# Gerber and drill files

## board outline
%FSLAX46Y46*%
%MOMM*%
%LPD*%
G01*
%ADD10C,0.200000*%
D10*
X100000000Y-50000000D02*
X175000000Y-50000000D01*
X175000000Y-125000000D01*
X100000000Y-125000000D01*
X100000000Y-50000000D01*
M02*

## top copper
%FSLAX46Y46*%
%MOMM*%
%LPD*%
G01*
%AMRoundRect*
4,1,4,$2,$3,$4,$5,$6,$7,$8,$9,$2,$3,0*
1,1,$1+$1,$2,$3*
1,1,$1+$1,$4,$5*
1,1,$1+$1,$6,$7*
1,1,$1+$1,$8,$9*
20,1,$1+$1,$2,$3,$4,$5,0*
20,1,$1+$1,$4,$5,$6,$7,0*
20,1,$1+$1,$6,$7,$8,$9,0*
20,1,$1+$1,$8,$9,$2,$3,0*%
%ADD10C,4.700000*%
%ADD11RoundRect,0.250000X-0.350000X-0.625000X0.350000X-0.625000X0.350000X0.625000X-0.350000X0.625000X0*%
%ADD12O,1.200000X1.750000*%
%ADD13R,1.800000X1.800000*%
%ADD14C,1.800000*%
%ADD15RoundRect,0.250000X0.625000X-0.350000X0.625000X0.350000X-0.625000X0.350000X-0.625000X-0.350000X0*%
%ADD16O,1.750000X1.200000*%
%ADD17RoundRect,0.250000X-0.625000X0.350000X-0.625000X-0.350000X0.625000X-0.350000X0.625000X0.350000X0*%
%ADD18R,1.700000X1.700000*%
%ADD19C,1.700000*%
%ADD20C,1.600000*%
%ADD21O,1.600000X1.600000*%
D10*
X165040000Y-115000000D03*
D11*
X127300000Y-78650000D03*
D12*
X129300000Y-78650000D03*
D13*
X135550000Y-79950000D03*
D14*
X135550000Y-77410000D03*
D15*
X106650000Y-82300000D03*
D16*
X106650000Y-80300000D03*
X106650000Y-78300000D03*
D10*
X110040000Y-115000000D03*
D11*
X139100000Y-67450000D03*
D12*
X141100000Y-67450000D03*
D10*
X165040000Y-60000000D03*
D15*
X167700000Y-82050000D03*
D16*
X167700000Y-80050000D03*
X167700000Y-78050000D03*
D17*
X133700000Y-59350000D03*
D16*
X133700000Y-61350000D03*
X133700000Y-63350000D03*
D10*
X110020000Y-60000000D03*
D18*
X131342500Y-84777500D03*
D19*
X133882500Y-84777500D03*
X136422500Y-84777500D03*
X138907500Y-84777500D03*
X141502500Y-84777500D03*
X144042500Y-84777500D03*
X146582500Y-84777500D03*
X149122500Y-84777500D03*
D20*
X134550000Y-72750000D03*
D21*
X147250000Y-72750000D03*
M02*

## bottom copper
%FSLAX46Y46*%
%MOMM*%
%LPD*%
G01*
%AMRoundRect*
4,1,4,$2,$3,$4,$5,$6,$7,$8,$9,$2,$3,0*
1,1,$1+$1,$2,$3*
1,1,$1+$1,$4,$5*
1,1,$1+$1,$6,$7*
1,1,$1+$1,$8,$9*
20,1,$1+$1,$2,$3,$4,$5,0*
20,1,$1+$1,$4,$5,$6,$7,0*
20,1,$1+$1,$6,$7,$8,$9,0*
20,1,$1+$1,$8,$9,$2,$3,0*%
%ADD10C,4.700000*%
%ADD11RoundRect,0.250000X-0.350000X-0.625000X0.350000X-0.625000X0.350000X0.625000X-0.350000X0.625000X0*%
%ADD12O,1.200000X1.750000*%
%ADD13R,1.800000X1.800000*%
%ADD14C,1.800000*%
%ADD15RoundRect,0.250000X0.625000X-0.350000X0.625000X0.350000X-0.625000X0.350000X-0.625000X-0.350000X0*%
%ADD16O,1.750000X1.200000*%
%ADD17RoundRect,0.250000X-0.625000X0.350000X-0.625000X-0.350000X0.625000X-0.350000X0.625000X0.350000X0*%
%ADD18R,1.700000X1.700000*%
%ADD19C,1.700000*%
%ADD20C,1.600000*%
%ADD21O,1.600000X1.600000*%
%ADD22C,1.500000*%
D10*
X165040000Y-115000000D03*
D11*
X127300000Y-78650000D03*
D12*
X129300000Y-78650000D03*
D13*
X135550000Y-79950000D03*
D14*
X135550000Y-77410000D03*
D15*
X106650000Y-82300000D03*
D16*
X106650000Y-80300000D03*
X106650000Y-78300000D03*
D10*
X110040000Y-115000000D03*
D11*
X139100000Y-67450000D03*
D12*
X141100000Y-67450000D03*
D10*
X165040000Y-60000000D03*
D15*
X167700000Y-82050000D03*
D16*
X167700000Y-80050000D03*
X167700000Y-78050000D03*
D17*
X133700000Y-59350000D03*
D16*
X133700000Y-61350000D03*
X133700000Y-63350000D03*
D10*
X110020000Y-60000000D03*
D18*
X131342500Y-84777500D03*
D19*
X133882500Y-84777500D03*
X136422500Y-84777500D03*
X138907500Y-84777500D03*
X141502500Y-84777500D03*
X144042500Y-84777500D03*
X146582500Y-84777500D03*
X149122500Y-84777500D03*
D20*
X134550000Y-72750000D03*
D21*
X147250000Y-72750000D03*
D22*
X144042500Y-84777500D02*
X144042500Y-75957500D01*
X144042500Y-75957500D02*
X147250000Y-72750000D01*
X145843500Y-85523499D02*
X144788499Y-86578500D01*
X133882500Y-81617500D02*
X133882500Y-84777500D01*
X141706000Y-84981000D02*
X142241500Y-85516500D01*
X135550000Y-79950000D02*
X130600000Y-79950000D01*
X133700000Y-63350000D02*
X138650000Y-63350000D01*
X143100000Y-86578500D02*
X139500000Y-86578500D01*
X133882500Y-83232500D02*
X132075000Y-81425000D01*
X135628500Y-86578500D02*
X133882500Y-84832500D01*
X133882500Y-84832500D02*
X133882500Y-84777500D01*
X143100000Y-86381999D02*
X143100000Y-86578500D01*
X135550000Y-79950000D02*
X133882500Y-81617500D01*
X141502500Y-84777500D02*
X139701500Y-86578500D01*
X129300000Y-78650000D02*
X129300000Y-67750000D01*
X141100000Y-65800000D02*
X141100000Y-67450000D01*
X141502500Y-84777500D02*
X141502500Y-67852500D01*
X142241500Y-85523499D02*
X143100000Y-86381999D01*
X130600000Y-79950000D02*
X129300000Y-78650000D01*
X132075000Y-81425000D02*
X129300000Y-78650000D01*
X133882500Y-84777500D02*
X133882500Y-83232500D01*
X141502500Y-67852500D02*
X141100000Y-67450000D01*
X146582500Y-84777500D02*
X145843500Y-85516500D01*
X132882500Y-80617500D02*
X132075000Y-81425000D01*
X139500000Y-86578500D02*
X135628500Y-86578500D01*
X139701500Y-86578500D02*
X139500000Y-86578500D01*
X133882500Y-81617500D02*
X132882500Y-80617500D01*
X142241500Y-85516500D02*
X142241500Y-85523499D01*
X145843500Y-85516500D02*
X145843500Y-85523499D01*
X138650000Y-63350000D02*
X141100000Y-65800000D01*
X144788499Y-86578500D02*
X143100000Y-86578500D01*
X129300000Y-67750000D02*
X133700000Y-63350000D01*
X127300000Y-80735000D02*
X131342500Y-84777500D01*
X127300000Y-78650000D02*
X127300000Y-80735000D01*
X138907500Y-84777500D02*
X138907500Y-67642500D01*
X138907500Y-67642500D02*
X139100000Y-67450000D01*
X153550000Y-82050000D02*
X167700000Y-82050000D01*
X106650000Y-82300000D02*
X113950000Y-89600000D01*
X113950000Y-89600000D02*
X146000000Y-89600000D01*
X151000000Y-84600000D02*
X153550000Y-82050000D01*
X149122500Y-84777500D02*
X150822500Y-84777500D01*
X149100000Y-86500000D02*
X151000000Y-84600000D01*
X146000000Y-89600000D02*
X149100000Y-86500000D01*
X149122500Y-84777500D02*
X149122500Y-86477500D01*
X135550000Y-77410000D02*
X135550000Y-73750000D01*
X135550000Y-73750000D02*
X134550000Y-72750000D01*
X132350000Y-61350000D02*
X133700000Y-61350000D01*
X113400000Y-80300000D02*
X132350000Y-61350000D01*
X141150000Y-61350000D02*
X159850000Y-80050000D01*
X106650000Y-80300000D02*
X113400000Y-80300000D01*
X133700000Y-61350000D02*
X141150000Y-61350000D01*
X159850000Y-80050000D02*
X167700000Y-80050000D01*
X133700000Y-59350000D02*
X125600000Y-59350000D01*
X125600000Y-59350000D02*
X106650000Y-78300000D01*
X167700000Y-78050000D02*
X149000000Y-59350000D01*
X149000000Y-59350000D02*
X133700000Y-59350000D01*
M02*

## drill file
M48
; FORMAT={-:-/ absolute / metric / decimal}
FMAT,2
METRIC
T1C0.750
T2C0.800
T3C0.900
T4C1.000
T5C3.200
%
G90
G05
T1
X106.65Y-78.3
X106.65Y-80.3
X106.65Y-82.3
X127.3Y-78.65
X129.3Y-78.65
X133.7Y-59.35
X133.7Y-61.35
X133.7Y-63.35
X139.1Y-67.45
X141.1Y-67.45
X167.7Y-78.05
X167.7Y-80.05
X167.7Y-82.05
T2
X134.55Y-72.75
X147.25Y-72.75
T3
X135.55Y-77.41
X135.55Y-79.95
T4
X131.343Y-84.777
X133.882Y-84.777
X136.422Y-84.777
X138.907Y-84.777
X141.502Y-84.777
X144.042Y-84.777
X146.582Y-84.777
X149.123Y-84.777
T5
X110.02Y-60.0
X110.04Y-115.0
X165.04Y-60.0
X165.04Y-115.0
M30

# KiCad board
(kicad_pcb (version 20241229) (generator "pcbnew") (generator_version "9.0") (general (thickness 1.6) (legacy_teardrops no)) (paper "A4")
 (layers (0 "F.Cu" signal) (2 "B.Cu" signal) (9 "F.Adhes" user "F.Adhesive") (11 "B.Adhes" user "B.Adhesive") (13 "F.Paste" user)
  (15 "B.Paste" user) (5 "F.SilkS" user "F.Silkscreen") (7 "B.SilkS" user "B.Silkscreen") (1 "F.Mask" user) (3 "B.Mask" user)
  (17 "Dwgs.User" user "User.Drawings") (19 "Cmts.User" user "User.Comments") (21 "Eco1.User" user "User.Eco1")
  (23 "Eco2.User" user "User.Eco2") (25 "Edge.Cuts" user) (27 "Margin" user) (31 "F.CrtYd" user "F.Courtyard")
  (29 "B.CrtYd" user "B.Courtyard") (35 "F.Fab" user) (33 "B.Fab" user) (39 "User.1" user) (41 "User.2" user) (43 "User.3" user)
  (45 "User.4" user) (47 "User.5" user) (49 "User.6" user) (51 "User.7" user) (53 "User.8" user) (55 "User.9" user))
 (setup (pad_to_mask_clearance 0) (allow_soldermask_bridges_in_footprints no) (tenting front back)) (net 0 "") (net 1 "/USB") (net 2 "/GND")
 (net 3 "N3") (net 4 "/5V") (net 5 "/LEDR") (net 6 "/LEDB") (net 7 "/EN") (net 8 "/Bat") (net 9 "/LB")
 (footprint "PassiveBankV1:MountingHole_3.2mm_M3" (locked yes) (layer "F.Cu") (at 165.02 115)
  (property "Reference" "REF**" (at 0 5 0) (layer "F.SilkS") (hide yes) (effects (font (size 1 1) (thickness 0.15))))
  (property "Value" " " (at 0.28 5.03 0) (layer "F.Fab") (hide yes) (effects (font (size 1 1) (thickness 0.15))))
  (pad "" np_thru_hole circle (at 0.02 0) (size 4.7 4.7) (drill 3.2) (layers "*.Cu" "*.Mask") (clearance 2)))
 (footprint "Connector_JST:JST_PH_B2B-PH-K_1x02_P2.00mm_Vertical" (layer "F.Cu") (at 127.3 78.65)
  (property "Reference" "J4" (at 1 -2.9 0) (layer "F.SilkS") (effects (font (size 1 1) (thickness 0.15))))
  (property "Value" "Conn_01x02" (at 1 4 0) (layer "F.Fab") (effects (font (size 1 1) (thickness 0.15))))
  (pad "1" thru_hole roundrect (at 0 0) (size 1.2 1.75) (drill 0.75) (layers "*.Cu" "*.Mask") (remove_unused_layers no)
   (roundrect_rratio 0.208333) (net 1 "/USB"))
  (pad "2" thru_hole oval (at 2 0) (size 1.2 1.75) (drill 0.75) (layers "*.Cu" "*.Mask") (remove_unused_layers no) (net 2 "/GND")))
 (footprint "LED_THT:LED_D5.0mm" (layer "F.Cu") (at 135.55 79.95 90)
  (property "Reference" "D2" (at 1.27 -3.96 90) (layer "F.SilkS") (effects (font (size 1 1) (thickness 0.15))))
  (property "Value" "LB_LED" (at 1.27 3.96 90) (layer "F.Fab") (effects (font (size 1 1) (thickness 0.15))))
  (pad "1" thru_hole rect (at 0 0 90) (size 1.8 1.8) (drill 0.9) (layers "*.Cu" "*.Mask") (remove_unused_layers no) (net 2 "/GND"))
  (pad "2" thru_hole circle (at 2.54 0 90) (size 1.8 1.8) (drill 0.9) (layers "*.Cu" "*.Mask") (remove_unused_layers no) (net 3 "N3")))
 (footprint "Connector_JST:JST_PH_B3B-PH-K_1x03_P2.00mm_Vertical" (layer "F.Cu") (at 106.65 82.3 90)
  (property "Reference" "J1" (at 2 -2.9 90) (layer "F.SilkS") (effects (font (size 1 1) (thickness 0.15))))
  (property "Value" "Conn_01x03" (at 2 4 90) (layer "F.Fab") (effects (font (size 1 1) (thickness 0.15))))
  (pad "1" thru_hole roundrect (at 0 0 90) (size 1.2 1.75) (drill 0.75) (layers "*.Cu" "*.Mask") (remove_unused_layers no)
   (roundrect_rratio 0.208333) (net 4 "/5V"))
  (pad "2" thru_hole oval (at 2 0 90) (size 1.2 1.75) (drill 0.75) (layers "*.Cu" "*.Mask") (remove_unused_layers no) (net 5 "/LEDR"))
  (pad "3" thru_hole oval (at 4 0 90) (size 1.2 1.75) (drill 0.75) (layers "*.Cu" "*.Mask") (remove_unused_layers no) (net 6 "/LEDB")))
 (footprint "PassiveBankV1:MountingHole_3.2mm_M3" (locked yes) (layer "F.Cu") (at 110.02 115)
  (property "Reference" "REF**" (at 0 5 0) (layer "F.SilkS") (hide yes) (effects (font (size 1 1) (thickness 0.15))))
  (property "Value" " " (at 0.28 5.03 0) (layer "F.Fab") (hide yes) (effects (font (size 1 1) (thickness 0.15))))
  (pad "" np_thru_hole circle (at 0.02 0) (size 4.7 4.7) (drill 3.2) (layers "*.Cu" "*.Mask") (clearance 2)))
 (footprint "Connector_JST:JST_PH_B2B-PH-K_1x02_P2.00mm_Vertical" (layer "F.Cu") (at 139.1 67.45)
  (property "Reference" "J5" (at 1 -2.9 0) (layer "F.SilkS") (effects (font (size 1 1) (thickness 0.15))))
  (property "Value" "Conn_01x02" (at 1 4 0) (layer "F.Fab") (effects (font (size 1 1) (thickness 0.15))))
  (pad "1" thru_hole roundrect (at 0 0) (size 1.2 1.75) (drill 0.75) (layers "*.Cu" "*.Mask") (remove_unused_layers no)
   (roundrect_rratio 0.208333) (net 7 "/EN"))
  (pad "2" thru_hole oval (at 2 0) (size 1.2 1.75) (drill 0.75) (layers "*.Cu" "*.Mask") (remove_unused_layers no) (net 2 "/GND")))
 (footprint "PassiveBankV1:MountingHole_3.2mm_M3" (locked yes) (layer "F.Cu") (at 165.02 60)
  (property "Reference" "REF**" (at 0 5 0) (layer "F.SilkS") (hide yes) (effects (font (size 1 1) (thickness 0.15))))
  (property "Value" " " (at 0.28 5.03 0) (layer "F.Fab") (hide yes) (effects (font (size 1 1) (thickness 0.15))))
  (pad "" np_thru_hole circle (at 0.02 0) (size 4.7 4.7) (drill 3.2) (layers "*.Cu" "*.Mask") (clearance 2)))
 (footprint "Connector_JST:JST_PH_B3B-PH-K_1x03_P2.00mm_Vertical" (layer "F.Cu") (at 167.7 82.05 90)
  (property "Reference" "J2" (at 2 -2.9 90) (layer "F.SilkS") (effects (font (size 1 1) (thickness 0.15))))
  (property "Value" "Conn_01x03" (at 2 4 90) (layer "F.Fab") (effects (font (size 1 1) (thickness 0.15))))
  (pad "1" thru_hole roundrect (at 0 0 90) (size 1.2 1.75) (drill 0.75) (layers "*.Cu" "*.Mask") (remove_unused_layers no)
   (roundrect_rratio 0.208333) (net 4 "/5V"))
  (pad "2" thru_hole oval (at 2 0 90) (size 1.2 1.75) (drill 0.75) (layers "*.Cu" "*.Mask") (remove_unused_layers no) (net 5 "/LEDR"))
  (pad "3" thru_hole oval (at 4 0 90) (size 1.2 1.75) (drill 0.75) (layers "*.Cu" "*.Mask") (remove_unused_layers no) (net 6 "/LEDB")))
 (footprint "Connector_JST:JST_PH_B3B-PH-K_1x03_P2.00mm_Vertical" (layer "F.Cu") (at 133.7 59.35 -90)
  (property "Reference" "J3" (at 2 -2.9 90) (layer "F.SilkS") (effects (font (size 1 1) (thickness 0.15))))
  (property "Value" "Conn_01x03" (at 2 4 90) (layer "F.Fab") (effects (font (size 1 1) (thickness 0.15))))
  (pad "1" thru_hole roundrect (at 0 0 270) (size 1.2 1.75) (drill 0.75) (layers "*.Cu" "*.Mask") (remove_unused_layers no)
   (roundrect_rratio 0.208333) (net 6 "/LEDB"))
  (pad "2" thru_hole oval (at 2 0 270) (size 1.2 1.75) (drill 0.75) (layers "*.Cu" "*.Mask") (remove_unused_layers no) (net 5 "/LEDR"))
  (pad "3" thru_hole oval (at 4 0 270) (size 1.2 1.75) (drill 0.75) (layers "*.Cu" "*.Mask") (remove_unused_layers no) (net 2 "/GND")))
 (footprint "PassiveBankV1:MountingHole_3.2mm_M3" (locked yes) (layer "F.Cu") (at 110 60)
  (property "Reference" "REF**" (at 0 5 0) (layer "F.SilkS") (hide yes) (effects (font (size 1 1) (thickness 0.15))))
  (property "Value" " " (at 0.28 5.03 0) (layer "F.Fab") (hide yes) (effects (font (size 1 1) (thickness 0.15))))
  (pad "" np_thru_hole circle (at 0.02 0) (size 4.7 4.7) (drill 3.2) (layers "*.Cu" "*.Mask") (clearance 2)))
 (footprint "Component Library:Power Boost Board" (layer "F.Cu") (at 149.1225 84.7775 -90)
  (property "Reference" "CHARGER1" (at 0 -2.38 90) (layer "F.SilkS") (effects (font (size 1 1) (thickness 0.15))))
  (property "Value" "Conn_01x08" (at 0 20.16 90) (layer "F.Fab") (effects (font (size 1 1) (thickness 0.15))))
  (pad "1" thru_hole rect (at 0 17.78 270) (size 1.7 1.7) (drill 1) (layers "*.Cu" "*.Mask") (remove_unused_layers no) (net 1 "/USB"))
  (pad "2" thru_hole circle (at 0 15.24 270) (size 1.7 1.7) (drill 1) (layers "*.Cu" "*.Mask") (remove_unused_layers no) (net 2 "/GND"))
  (pad "3" thru_hole circle (at 0 12.7 270) (size 1.7 1.7) (drill 1) (layers "*.Cu" "*.Mask") (remove_unused_layers no) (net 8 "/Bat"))
  (pad "4" thru_hole circle (at 0 10.215 270) (size 1.7 1.7) (drill 1) (layers "*.Cu" "*.Mask") (remove_unused_layers no) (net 7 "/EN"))
  (pad "5" thru_hole circle (at 0 7.62 270) (size 1.7 1.7) (drill 1) (layers "*.Cu" "*.Mask") (remove_unused_layers no) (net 2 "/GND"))
  (pad "6" thru_hole circle (at 0 5.08 270) (size 1.7 1.7) (drill 1) (layers "*.Cu" "*.Mask") (remove_unused_layers no) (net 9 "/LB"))
  (pad "7" thru_hole circle (at 0 2.54 270) (size 1.7 1.7) (drill 1) (layers "*.Cu" "*.Mask") (remove_unused_layers no) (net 2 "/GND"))
  (pad "8" thru_hole circle (at 0 0 270) (size 1.7 1.7) (drill 1) (layers "*.Cu" "*.Mask") (remove_unused_layers no) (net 4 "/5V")))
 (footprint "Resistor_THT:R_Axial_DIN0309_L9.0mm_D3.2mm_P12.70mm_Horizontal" (layer "F.Cu") (at 134.55 72.75)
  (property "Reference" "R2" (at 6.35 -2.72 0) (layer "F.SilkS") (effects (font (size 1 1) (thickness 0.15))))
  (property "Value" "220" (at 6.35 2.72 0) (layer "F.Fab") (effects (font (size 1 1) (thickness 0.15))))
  (pad "1" thru_hole circle (at 0 0) (size 1.6 1.6) (drill 0.8) (layers "*.Cu" "*.Mask") (remove_unused_layers no) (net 3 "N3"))
  (pad "2" thru_hole oval (at 12.7 0) (size 1.6 1.6) (drill 0.8) (layers "*.Cu" "*.Mask") (remove_unused_layers no) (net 9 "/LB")))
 (gr_rect (start 100 50) (end 175 125) (stroke (width 0.2) (type default)) (fill no) (locked yes) (layer "Edge.Cuts"))
 (segment (start 144.0425 84.7775) (end 144.0425 75.9575) (width 1.5) (layer "B.Cu") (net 9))
 (segment (start 144.0425 75.9575) (end 147.25 72.75) (width 1.5) (layer "B.Cu") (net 9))
 (segment (start 145.8435 85.523499) (end 144.788499 86.5785) (width 1.5) (layer "B.Cu") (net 2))
 (segment (start 133.8825 81.6175) (end 133.8825 84.7775) (width 1.5) (layer "B.Cu") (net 2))
 (segment (start 141.706 84.981) (end 142.2415 85.5165) (width 1.5) (layer "B.Cu") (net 2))
 (segment (start 135.55 79.95) (end 130.6 79.95) (width 1.5) (layer "B.Cu") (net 2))
 (segment (start 133.7 63.35) (end 138.65 63.35) (width 1.5) (layer "B.Cu") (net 2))
 (segment (start 143.1 86.5785) (end 139.5 86.5785) (width 1.5) (layer "B.Cu") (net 2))
 (segment (start 133.8825 83.2325) (end 132.075 81.425) (width 1.5) (layer "B.Cu") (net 2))
 (segment (start 135.6285 86.5785) (end 133.8825 84.8325) (width 1.5) (layer "B.Cu") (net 2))
 (segment (start 133.8825 84.8325) (end 133.8825 84.7775) (width 1.5) (layer "B.Cu") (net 2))
 (segment (start 143.1 86.381999) (end 143.1 86.5785) (width 1.5) (layer "B.Cu") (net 2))
 (segment (start 135.55 79.95) (end 133.8825 81.6175) (width 1.5) (layer "B.Cu") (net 2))
 (segment (start 141.5025 84.7775) (end 139.7015 86.5785) (width 1.5) (layer "B.Cu") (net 2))
 (segment (start 129.3 78.65) (end 129.3 67.75) (width 1.5) (layer "B.Cu") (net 2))
 (segment (start 141.1 65.8) (end 141.1 67.45) (width 1.5) (layer "B.Cu") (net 2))
 (segment (start 141.5025 84.7775) (end 141.5025 67.8525) (width 1.5) (layer "B.Cu") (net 2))
 (segment (start 142.2415 85.523499) (end 143.1 86.381999) (width 1.5) (layer "B.Cu") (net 2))
 (segment (start 130.6 79.95) (end 129.3 78.65) (width 1.5) (layer "B.Cu") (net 2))
 (segment (start 132.075 81.425) (end 129.3 78.65) (width 1.5) (layer "B.Cu") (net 2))
 (segment (start 133.8825 84.7775) (end 133.8825 83.2325) (width 1.5) (layer "B.Cu") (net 2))
 (segment (start 141.5025 67.8525) (end 141.1 67.45) (width 1.5) (layer "B.Cu") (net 2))
 (segment (start 146.5825 84.7775) (end 145.8435 85.5165) (width 1.5) (layer "B.Cu") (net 2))
 (segment (start 132.8825 80.6175) (end 132.075 81.425) (width 1.5) (layer "B.Cu") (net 2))
 (segment (start 139.5 86.5785) (end 135.6285 86.5785) (width 1.5) (layer "B.Cu") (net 2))
 (segment (start 139.7015 86.5785) (end 139.5 86.5785) (width 1.5) (layer "B.Cu") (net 2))
 (segment (start 133.8825 81.6175) (end 132.8825 80.6175) (width 1.5) (layer "B.Cu") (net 2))
 (segment (start 142.2415 85.5165) (end 142.2415 85.523499) (width 1.5) (layer "B.Cu") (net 2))
 (segment (start 145.8435 85.5165) (end 145.8435 85.523499) (width 1.5) (layer "B.Cu") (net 2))
 (segment (start 138.65 63.35) (end 141.1 65.8) (width 1.5) (layer "B.Cu") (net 2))
 (segment (start 144.788499 86.5785) (end 143.1 86.5785) (width 1.5) (layer "B.Cu") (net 2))
 (segment (start 129.3 67.75) (end 133.7 63.35) (width 1.5) (layer "B.Cu") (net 2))
 (segment (start 127.3 80.735) (end 131.3425 84.7775) (width 1.5) (layer "B.Cu") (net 1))
 (segment (start 127.3 78.65) (end 127.3 80.735) (width 1.5) (layer "B.Cu") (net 1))
 (segment (start 138.9075 84.7775) (end 138.9075 67.6425) (width 1.5) (layer "B.Cu") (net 7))
 (segment (start 138.9075 67.6425) (end 139.1 67.45) (width 1.5) (layer "B.Cu") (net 7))
 (segment (start 153.55 82.05) (end 167.7 82.05) (width 1.5) (layer "B.Cu") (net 4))
 (segment (start 106.65 82.3) (end 113.95 89.6) (width 1.5) (layer "B.Cu") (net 4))
 (segment (start 113.95 89.6) (end 146 89.6) (width 1.5) (layer "B.Cu") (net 4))
 (segment (start 151 84.6) (end 153.55 82.05) (width 1.5) (layer "B.Cu") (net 4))
 (segment (start 149.1225 84.7775) (end 150.8225 84.7775) (width 1.5) (layer "B.Cu") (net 4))
 (segment (start 149.1 86.5) (end 151 84.6) (width 1.5) (layer "B.Cu") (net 4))
 (segment (start 146 89.6) (end 149.1 86.5) (width 1.5) (layer "B.Cu") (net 4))
 (segment (start 149.1225 84.7775) (end 149.1225 86.4775) (width 1.5) (layer "B.Cu") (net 4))
 (segment (start 135.55 77.41) (end 135.55 73.75) (width 1.5) (layer "B.Cu") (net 3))
 (segment (start 135.55 73.75) (end 134.55 72.75) (width 1.5) (layer "B.Cu") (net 3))
 (segment (start 132.35 61.35) (end 133.7 61.35) (width 1.5) (layer "B.Cu") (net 5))
 (segment (start 113.4 80.3) (end 132.35 61.35) (width 1.5) (layer "B.Cu") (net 5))
 (segment (start 141.15 61.35) (end 159.85 80.05) (width 1.5) (layer "B.Cu") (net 5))
 (segment (start 106.65 80.3) (end 113.4 80.3) (width 1.5) (layer "B.Cu") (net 5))
 (segment (start 133.7 61.35) (end 141.15 61.35) (width 1.5) (layer "B.Cu") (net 5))
 (segment (start 159.85 80.05) (end 167.7 80.05) (width 1.5) (layer "B.Cu") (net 5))
 (segment (start 133.7 59.35) (end 125.6 59.35) (width 1.5) (layer "B.Cu") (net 6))
 (segment (start 125.6 59.35) (end 106.65 78.3) (width 1.5) (layer "B.Cu") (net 6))
 (segment (start 167.7 78.05) (end 149 59.35) (width 1.5) (layer "B.Cu") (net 6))
 (segment (start 149 59.35) (end 133.7 59.35) (width 1.5) (layer "B.Cu") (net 6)))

